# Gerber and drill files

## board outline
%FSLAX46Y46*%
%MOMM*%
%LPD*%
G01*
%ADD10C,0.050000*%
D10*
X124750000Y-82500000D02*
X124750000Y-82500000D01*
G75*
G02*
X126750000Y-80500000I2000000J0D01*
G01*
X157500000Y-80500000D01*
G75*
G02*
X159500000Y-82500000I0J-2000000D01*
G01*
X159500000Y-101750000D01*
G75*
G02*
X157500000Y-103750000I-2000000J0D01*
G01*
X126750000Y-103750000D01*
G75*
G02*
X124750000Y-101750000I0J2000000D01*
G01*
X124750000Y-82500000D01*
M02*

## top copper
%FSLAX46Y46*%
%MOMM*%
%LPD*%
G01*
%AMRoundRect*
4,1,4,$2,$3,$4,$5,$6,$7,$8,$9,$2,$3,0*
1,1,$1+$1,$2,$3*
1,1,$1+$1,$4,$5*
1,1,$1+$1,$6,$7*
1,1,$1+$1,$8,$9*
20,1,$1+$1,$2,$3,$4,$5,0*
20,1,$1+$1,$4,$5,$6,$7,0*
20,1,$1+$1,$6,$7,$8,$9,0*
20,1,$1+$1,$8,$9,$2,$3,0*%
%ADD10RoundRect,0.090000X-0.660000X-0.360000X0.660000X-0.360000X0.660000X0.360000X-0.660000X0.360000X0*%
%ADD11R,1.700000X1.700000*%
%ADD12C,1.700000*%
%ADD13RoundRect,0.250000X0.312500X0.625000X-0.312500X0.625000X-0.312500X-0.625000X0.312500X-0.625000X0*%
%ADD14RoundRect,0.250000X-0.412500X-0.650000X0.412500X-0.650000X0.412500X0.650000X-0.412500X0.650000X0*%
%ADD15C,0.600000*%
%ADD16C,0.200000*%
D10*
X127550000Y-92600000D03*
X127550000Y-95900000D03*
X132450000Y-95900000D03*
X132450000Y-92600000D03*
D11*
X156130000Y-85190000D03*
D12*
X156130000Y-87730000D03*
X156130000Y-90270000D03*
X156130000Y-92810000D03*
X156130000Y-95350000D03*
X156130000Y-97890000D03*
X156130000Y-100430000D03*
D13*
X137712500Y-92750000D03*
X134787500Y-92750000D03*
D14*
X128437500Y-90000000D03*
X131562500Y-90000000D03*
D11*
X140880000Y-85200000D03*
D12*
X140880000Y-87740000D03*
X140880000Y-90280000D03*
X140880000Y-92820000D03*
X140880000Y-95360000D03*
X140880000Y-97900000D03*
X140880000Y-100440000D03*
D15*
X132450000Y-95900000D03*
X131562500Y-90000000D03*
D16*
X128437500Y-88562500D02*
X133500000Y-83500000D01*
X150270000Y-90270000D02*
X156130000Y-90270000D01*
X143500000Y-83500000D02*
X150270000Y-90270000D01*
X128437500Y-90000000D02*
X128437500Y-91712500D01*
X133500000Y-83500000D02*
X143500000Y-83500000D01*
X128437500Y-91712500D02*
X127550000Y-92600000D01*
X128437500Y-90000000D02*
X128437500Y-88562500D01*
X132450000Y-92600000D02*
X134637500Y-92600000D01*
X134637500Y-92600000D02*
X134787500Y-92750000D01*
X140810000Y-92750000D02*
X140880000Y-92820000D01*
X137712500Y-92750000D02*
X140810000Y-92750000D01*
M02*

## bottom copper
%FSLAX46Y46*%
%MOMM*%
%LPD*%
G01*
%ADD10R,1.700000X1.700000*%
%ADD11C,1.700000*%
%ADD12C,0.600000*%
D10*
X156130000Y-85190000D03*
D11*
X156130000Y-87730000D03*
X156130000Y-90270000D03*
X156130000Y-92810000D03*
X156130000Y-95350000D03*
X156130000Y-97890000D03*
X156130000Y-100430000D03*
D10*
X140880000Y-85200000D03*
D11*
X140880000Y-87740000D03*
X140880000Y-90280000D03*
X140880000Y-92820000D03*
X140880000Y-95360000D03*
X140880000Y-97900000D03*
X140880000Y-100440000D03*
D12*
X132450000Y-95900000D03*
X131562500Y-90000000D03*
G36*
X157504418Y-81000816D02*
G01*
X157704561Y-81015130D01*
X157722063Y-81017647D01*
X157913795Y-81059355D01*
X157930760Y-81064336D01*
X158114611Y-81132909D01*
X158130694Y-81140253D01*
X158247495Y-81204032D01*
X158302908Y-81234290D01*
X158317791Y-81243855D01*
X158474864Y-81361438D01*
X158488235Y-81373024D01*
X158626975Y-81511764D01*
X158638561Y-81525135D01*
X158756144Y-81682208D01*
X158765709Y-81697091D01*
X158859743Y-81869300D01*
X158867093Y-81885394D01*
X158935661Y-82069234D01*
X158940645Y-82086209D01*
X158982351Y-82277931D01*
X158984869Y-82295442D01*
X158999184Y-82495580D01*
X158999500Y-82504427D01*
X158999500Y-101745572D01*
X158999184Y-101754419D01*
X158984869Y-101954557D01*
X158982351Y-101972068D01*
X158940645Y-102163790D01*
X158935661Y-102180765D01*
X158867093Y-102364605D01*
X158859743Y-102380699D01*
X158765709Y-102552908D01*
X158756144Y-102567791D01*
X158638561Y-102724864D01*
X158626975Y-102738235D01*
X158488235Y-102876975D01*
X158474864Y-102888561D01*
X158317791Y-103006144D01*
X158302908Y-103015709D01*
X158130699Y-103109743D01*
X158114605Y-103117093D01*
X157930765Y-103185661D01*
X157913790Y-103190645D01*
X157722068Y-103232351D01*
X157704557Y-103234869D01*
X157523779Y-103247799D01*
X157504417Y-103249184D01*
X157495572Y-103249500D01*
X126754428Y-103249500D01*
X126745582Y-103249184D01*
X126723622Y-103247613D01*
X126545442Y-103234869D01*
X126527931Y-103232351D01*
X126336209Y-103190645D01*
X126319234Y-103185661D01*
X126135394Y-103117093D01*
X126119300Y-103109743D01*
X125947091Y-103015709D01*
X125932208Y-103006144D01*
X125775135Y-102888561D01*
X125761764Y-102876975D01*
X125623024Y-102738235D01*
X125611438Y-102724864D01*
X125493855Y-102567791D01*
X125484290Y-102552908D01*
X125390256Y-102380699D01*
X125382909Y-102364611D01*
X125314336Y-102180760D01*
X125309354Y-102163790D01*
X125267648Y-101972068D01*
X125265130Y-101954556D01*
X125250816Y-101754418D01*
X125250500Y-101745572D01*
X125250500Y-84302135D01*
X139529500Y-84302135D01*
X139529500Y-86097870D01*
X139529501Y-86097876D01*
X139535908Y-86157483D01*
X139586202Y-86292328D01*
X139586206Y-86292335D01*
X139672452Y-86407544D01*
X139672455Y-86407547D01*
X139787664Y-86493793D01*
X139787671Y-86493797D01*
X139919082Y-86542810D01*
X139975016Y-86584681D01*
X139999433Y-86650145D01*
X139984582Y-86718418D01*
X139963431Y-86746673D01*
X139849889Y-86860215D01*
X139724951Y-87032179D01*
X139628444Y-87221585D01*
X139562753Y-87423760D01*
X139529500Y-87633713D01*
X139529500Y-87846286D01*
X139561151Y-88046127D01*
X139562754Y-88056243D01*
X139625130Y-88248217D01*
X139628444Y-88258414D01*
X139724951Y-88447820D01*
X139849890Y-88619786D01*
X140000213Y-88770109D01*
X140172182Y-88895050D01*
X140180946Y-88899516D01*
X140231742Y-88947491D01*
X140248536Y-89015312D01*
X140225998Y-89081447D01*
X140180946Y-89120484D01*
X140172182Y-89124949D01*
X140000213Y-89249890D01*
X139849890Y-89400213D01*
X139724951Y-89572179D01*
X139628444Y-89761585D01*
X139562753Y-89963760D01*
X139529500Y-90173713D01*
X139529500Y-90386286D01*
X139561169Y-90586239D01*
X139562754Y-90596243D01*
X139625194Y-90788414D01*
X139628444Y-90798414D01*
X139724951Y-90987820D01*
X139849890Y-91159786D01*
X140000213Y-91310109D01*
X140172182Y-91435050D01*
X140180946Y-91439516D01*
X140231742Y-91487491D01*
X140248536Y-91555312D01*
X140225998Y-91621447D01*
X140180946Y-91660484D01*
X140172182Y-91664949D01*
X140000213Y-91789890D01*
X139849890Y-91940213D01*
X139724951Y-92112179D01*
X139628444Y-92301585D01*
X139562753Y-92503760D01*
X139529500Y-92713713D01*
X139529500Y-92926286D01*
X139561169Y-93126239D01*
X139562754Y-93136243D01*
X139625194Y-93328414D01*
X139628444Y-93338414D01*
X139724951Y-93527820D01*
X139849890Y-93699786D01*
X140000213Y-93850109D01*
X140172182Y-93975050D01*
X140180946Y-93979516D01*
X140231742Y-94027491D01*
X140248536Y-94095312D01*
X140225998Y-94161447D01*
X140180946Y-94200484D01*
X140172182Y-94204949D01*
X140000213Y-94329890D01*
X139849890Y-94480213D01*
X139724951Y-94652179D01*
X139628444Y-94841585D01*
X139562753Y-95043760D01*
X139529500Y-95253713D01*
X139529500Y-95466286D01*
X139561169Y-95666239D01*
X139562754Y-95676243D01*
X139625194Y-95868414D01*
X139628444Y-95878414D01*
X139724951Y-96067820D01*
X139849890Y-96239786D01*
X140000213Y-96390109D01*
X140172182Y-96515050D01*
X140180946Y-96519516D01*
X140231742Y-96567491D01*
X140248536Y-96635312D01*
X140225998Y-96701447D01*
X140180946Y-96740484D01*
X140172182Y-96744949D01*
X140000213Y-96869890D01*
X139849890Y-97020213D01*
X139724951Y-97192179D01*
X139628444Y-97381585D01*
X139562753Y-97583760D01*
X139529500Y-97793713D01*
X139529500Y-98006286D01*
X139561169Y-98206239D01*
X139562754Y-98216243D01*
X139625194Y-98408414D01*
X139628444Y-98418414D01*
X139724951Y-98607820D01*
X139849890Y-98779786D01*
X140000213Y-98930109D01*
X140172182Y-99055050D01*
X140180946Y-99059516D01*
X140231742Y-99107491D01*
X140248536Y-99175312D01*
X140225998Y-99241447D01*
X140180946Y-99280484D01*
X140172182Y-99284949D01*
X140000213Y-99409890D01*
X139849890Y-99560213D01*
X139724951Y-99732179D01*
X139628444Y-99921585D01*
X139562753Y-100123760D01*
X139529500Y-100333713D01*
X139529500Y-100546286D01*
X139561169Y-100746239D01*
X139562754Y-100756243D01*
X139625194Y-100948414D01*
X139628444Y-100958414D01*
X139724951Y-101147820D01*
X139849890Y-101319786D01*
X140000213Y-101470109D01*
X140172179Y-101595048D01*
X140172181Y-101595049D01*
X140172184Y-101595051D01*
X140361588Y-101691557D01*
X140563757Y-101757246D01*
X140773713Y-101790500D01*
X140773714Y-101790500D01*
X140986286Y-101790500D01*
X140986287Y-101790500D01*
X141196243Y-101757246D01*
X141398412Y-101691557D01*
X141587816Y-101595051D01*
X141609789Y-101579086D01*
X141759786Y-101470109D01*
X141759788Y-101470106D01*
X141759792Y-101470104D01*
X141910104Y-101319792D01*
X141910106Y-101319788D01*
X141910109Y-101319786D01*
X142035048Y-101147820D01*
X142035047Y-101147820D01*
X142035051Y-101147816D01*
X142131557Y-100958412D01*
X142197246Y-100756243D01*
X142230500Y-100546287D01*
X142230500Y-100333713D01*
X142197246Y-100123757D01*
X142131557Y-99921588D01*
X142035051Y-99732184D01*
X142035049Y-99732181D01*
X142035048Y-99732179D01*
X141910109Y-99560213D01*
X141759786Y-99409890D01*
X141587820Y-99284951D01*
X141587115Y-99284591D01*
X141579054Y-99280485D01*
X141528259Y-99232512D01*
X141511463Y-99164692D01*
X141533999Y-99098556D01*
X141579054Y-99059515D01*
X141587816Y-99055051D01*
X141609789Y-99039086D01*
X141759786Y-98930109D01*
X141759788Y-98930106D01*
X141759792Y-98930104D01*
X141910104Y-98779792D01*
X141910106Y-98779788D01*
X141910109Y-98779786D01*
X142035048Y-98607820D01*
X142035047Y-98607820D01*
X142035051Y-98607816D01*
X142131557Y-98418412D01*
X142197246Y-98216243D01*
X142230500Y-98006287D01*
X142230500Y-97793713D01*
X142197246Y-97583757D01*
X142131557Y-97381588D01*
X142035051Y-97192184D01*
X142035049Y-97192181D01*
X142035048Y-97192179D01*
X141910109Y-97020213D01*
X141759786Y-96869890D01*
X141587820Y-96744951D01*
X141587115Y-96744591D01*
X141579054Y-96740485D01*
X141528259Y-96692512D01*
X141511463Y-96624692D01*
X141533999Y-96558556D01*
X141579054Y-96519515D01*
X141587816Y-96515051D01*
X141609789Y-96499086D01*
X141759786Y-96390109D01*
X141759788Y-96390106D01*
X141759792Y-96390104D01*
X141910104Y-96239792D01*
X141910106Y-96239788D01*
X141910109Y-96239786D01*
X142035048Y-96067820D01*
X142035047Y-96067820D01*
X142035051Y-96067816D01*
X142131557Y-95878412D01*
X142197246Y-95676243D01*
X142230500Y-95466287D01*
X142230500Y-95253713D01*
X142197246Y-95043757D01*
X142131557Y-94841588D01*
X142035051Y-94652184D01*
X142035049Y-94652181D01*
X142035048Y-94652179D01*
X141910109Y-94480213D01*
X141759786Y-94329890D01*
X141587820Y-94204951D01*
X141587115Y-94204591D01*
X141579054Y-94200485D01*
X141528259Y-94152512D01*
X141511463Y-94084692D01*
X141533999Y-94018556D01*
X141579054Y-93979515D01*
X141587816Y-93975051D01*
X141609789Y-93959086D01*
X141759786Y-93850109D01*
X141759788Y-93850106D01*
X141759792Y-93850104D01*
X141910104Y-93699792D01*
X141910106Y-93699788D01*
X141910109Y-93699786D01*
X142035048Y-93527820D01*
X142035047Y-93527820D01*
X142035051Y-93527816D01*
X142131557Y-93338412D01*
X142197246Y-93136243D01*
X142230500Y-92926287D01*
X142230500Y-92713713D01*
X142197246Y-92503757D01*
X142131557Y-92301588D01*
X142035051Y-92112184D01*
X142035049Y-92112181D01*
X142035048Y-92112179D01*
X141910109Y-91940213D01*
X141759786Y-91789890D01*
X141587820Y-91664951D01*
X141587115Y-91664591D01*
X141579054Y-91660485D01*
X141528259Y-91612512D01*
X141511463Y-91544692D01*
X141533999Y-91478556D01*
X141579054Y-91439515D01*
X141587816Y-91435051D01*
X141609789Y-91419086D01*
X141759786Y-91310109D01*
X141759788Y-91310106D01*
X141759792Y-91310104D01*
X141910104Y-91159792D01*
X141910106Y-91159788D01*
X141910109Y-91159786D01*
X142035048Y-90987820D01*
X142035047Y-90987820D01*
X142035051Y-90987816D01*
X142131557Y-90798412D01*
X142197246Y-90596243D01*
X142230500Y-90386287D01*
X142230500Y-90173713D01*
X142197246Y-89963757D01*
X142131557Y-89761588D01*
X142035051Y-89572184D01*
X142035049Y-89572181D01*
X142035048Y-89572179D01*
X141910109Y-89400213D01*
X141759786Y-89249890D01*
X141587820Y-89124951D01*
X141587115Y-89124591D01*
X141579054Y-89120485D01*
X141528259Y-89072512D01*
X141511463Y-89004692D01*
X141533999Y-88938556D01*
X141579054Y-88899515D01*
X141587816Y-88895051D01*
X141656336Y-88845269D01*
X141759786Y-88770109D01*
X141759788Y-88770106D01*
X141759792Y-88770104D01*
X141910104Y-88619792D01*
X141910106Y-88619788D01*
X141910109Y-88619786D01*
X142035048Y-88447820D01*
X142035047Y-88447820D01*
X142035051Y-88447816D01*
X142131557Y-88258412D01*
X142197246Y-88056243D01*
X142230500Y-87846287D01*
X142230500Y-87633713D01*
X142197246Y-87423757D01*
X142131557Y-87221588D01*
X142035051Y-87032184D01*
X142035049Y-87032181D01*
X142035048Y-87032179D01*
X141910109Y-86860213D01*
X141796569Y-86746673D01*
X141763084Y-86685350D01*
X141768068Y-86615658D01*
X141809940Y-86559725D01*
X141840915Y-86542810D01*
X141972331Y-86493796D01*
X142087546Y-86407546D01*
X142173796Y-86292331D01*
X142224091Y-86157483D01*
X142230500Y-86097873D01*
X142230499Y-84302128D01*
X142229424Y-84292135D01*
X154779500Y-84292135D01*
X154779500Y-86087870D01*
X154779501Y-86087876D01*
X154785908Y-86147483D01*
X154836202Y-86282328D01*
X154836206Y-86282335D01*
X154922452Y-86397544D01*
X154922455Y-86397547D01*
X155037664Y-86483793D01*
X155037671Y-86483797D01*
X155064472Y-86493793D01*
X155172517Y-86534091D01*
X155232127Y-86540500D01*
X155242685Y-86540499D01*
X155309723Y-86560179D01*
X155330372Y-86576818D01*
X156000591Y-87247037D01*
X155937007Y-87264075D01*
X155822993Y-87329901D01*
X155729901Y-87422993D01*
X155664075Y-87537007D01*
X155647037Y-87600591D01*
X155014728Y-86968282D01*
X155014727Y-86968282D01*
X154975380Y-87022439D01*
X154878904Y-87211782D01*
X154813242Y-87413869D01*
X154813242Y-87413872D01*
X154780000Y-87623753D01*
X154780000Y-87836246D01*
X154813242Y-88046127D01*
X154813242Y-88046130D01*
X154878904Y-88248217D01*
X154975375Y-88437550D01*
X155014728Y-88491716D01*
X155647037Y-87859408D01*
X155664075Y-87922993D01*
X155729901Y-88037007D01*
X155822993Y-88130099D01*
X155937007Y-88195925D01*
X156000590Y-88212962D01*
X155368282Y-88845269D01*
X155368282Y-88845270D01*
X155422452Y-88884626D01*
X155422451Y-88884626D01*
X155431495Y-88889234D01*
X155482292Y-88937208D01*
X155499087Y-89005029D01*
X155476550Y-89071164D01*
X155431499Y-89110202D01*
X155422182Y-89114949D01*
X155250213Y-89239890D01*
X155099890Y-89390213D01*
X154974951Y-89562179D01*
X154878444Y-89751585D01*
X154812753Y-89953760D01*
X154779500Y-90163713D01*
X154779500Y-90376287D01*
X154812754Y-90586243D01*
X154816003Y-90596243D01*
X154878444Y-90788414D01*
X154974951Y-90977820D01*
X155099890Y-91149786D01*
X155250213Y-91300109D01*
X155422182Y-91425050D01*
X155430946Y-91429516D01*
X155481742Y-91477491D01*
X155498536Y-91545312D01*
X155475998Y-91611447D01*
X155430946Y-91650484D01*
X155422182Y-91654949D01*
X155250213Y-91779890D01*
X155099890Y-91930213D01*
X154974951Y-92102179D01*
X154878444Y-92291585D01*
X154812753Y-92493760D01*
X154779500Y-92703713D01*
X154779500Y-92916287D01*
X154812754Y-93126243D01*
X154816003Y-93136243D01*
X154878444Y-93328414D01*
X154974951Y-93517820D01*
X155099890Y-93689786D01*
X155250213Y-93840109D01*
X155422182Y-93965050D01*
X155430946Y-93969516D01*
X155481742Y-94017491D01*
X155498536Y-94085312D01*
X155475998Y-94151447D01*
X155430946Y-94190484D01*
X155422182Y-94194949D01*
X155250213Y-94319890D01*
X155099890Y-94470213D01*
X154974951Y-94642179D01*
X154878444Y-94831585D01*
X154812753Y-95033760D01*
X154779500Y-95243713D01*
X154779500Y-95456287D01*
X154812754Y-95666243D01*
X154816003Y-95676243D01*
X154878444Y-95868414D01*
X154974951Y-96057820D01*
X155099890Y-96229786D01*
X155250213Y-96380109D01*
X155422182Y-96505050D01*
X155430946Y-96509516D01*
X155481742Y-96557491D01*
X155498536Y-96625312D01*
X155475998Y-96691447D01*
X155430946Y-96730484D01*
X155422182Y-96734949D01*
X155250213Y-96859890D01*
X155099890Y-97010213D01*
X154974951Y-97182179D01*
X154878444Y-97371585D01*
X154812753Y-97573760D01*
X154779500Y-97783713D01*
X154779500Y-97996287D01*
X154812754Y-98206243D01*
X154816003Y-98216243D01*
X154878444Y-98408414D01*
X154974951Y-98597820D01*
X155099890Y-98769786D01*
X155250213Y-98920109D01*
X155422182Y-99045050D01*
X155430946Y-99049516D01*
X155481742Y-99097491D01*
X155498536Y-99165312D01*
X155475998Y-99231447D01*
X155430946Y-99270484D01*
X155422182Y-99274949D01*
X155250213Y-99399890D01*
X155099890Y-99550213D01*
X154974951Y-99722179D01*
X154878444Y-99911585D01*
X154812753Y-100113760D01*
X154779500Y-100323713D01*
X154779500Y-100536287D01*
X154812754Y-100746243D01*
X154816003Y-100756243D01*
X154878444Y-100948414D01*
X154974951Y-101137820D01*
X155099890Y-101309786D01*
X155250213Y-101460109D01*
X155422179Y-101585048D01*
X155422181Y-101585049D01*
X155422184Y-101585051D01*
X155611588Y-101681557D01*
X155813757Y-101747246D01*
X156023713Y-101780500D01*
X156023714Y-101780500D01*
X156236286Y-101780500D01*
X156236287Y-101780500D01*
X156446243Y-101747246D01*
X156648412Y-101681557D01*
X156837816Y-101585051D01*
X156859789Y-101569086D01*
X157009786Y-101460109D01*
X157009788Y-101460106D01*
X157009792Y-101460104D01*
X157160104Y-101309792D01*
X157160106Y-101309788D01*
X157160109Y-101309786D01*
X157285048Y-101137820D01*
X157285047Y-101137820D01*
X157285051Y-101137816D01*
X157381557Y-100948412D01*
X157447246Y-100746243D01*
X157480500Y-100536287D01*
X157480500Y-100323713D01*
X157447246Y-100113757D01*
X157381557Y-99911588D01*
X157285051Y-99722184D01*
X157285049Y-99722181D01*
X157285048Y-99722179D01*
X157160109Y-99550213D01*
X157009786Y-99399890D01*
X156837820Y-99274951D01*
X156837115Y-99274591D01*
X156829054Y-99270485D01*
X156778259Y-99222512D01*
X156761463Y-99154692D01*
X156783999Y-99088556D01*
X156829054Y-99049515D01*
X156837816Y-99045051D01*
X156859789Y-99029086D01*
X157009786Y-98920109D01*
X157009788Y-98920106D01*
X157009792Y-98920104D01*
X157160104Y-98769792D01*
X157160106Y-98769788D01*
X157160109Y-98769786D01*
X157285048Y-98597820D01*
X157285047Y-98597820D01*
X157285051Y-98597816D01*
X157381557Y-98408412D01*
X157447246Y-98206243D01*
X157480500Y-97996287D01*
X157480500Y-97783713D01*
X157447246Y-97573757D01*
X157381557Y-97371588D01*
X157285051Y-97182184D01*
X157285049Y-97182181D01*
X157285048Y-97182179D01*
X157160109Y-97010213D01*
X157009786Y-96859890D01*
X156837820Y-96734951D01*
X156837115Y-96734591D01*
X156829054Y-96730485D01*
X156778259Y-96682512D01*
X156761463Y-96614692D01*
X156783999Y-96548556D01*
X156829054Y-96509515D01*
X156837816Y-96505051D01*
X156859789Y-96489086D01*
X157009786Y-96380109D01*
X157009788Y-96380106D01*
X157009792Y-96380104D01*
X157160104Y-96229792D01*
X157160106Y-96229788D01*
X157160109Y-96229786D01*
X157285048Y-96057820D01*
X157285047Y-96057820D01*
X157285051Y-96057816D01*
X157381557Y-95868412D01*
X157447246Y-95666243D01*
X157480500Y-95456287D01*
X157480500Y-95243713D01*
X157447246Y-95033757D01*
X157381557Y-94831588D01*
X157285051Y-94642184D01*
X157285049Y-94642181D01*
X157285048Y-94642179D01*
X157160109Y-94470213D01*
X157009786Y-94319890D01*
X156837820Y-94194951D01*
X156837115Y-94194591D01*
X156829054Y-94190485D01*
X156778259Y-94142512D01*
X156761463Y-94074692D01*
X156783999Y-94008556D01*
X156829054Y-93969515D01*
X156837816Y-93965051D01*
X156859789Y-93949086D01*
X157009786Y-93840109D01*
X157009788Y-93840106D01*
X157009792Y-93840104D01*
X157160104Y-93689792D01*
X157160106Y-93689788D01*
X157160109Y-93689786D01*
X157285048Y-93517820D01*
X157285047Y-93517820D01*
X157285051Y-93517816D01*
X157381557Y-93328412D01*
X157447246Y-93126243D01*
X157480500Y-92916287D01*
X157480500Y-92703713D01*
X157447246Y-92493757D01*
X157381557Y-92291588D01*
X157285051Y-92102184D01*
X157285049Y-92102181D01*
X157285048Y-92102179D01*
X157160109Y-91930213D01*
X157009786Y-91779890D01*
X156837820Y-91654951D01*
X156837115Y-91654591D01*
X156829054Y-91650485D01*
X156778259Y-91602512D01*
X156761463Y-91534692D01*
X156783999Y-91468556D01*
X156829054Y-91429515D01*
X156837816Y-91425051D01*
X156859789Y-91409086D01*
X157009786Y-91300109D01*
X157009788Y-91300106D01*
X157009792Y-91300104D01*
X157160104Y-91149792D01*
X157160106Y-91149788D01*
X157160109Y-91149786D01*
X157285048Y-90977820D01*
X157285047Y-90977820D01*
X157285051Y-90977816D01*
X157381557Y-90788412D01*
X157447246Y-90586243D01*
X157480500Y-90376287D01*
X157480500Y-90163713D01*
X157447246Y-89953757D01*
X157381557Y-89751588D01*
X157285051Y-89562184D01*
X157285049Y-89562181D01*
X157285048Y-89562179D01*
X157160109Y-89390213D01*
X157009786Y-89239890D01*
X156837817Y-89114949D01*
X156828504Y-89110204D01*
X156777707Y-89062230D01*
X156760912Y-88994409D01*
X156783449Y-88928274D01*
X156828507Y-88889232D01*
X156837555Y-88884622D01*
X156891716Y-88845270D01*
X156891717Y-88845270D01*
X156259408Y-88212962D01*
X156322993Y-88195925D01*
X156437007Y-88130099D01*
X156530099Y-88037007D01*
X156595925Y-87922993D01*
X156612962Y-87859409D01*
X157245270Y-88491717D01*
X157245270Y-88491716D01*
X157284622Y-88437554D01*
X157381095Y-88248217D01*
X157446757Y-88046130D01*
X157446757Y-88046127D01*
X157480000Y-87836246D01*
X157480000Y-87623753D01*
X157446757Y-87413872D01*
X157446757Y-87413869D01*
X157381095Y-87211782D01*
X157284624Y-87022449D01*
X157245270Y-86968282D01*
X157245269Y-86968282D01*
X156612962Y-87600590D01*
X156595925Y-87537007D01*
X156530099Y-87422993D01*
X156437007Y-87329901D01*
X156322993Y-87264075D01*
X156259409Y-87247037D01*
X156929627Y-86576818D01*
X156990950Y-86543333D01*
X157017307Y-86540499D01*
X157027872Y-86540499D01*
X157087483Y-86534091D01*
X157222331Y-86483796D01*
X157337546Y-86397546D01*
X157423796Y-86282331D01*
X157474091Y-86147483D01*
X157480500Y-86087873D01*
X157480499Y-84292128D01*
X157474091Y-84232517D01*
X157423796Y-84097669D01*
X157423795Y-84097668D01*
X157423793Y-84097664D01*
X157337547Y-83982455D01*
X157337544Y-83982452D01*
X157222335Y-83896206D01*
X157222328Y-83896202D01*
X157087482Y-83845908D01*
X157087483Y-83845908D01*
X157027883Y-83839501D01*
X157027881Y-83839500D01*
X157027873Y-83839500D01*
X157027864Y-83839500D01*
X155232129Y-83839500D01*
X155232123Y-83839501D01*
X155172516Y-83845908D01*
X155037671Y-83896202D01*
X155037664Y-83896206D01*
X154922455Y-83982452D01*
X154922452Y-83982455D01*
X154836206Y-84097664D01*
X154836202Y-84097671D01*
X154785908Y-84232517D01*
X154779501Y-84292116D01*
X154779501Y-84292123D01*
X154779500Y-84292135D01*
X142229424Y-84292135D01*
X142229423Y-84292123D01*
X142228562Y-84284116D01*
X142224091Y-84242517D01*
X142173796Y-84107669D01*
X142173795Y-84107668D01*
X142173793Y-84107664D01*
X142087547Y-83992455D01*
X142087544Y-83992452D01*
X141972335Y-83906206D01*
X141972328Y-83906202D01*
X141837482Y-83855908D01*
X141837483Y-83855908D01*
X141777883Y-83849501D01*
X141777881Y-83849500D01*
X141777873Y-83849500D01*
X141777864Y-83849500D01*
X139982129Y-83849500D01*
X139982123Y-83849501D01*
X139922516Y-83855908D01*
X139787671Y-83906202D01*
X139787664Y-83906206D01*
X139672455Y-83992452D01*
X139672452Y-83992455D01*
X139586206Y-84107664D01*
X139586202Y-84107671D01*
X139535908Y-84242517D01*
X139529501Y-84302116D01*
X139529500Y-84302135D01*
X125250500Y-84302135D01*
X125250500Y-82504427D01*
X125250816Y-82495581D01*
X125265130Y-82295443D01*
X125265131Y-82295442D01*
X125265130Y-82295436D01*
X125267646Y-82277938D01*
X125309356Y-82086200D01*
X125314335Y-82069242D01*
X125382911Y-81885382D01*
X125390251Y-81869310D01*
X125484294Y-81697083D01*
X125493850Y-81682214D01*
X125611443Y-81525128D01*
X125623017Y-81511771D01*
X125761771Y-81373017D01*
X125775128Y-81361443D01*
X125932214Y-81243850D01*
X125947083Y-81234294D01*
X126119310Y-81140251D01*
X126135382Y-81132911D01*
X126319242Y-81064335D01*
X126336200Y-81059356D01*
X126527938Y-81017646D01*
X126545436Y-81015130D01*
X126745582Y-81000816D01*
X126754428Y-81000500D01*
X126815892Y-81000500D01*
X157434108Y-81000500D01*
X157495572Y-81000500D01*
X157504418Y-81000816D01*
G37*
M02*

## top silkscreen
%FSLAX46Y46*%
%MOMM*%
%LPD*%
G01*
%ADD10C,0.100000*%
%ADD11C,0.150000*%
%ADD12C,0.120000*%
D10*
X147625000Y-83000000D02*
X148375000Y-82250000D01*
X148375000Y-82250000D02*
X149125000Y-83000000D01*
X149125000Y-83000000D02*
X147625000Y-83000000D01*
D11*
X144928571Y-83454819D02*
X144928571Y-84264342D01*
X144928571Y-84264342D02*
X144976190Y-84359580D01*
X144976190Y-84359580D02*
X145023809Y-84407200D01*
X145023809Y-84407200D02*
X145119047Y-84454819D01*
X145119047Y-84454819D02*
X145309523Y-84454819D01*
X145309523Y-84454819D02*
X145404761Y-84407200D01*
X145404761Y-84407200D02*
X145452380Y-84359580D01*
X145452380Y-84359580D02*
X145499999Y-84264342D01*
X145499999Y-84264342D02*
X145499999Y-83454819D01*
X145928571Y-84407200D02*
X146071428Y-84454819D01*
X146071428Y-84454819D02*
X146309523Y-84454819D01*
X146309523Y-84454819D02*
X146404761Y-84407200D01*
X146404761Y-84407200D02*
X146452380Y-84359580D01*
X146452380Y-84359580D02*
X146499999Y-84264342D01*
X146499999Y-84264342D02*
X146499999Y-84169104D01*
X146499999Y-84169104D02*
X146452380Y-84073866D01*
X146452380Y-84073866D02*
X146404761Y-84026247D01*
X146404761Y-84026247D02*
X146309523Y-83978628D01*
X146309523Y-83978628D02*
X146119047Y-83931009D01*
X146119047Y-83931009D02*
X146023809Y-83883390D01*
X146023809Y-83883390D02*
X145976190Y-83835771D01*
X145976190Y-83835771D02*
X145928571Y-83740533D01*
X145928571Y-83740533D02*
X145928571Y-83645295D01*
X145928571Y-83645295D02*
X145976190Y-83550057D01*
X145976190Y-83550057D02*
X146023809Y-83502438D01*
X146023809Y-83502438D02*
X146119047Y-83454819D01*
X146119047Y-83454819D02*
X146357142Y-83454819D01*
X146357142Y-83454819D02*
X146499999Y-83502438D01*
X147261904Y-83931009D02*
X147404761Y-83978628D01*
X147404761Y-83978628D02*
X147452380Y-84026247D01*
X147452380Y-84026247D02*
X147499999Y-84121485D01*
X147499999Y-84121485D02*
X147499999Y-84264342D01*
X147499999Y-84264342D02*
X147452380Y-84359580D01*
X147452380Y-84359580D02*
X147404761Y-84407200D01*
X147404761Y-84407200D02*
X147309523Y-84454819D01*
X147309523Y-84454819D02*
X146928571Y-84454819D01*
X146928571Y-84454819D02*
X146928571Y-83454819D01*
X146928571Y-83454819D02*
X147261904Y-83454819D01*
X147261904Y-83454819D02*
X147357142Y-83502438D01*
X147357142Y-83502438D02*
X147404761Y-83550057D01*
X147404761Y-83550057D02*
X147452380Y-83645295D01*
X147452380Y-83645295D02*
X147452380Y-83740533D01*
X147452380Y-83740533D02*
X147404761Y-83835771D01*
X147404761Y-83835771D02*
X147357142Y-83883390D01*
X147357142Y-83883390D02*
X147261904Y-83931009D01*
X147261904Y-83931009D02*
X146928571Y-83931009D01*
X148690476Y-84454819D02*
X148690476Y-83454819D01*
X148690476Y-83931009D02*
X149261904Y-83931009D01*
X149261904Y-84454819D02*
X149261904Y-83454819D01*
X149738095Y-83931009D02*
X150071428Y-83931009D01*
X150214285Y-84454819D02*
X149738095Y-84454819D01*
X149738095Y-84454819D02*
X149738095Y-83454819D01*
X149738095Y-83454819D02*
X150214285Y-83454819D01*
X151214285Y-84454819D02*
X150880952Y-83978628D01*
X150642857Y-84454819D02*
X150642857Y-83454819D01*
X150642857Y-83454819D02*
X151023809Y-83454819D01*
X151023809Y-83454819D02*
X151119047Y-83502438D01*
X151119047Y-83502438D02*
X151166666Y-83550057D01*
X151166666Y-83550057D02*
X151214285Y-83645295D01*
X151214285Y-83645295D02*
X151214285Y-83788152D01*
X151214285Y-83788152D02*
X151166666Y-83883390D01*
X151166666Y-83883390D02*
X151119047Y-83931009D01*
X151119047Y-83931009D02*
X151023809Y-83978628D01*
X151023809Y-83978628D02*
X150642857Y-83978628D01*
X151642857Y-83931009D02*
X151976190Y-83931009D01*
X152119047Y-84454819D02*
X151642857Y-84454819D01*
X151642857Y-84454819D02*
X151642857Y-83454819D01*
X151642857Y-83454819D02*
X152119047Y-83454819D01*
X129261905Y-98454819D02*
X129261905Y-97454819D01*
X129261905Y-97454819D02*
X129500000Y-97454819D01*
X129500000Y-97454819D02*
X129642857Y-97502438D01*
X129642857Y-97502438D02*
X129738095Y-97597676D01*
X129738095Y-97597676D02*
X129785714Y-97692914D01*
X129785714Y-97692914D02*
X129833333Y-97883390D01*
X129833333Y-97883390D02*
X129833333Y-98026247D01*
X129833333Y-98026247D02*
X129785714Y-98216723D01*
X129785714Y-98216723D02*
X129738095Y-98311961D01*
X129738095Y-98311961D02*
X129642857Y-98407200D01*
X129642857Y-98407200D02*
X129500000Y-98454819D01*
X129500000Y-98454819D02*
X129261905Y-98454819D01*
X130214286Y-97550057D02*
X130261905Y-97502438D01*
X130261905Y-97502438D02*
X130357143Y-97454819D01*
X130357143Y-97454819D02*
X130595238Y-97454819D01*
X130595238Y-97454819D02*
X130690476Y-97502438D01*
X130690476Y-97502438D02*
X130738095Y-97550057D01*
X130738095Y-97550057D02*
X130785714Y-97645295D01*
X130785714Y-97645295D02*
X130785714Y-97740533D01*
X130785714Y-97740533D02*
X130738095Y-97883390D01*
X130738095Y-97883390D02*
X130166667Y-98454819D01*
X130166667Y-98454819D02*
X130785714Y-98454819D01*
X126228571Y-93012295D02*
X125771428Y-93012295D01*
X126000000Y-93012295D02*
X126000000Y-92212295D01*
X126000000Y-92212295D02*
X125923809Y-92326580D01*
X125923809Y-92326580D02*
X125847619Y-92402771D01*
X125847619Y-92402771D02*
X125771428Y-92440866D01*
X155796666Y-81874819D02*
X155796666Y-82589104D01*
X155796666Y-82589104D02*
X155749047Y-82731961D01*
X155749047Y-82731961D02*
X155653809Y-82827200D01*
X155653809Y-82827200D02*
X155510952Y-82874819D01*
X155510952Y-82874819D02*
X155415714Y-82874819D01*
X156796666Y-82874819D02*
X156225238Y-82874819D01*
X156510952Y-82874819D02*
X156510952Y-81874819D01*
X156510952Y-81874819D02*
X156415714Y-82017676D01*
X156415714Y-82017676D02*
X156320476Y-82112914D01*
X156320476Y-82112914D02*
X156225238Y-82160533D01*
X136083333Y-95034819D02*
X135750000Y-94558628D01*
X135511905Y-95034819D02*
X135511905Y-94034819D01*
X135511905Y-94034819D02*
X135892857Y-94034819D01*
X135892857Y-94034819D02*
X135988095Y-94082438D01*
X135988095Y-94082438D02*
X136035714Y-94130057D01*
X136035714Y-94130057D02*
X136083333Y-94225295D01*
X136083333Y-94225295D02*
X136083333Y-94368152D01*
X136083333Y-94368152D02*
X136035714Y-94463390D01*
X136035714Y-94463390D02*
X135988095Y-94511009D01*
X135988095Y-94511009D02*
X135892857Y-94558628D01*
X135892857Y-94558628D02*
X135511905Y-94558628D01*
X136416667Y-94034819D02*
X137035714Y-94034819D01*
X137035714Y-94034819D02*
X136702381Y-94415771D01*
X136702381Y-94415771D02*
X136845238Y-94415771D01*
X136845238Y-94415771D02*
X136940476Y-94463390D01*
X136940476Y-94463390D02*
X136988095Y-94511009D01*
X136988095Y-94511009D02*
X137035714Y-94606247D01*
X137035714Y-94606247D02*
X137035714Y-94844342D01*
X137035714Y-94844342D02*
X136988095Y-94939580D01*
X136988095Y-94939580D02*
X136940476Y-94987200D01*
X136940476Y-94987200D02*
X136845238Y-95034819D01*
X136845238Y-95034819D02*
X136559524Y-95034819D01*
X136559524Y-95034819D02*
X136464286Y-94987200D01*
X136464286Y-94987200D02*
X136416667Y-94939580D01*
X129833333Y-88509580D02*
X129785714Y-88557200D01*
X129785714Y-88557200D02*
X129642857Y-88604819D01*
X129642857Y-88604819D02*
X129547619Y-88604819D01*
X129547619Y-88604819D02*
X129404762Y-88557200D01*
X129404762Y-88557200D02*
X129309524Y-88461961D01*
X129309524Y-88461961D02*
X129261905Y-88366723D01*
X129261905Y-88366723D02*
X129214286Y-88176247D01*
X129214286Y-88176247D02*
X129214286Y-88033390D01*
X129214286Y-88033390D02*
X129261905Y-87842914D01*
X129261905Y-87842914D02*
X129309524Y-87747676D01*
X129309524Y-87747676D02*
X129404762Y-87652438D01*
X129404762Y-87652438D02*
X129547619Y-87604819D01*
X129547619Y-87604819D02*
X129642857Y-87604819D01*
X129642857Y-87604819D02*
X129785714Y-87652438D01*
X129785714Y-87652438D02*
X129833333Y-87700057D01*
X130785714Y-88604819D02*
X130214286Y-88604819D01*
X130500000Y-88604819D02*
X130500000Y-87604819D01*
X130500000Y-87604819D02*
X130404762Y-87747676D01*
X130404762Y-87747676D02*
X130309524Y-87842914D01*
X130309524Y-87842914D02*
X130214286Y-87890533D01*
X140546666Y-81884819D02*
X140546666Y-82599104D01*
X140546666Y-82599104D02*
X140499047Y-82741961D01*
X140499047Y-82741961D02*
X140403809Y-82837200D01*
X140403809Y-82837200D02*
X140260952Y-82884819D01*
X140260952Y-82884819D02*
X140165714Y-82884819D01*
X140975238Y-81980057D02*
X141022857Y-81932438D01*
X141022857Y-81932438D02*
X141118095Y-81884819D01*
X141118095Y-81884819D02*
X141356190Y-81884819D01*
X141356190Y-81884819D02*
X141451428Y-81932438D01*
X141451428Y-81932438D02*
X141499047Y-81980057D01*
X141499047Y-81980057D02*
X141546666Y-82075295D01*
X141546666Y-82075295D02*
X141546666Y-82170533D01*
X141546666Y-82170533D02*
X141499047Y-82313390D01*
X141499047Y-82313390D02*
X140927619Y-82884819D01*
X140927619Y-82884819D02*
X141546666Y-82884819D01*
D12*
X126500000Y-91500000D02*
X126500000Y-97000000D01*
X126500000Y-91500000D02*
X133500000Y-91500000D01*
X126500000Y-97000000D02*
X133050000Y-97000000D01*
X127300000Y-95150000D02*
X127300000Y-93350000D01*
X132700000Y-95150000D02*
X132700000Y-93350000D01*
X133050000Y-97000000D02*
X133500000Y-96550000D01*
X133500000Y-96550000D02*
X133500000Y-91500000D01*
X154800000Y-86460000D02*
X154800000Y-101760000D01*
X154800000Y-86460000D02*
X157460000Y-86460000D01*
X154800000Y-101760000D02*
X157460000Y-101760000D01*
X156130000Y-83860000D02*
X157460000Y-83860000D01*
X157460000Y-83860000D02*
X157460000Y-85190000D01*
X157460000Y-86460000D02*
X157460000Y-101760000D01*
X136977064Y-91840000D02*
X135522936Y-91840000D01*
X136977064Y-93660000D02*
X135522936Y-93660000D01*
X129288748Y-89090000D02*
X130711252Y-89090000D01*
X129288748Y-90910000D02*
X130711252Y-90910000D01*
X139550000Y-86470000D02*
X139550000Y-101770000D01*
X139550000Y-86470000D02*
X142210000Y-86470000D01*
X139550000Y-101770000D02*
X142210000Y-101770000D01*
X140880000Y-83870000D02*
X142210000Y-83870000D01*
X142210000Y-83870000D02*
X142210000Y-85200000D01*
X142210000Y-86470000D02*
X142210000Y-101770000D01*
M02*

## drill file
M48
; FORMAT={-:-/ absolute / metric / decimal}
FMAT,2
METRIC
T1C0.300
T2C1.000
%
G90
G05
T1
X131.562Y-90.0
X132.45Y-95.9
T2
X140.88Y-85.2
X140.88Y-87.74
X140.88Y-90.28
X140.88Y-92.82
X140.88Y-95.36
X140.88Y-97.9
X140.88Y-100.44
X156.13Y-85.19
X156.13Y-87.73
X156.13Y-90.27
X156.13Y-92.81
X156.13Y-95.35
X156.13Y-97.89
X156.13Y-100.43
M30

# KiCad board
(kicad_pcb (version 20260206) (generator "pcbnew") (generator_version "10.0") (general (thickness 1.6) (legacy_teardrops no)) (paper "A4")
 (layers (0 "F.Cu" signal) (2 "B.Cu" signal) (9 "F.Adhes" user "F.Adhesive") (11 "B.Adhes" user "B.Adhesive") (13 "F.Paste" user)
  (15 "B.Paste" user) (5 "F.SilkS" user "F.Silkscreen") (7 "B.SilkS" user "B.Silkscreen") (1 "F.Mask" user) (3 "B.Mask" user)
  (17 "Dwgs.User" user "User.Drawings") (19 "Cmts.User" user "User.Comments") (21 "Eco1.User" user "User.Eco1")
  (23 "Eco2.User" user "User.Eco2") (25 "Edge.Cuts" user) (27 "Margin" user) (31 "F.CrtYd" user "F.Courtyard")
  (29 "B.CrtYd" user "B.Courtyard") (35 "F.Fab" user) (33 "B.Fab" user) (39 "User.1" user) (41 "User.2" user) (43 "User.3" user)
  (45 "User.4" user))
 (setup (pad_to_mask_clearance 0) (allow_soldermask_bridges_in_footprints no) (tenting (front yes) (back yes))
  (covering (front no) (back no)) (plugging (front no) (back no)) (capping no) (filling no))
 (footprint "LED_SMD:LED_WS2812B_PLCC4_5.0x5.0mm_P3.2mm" (layer "F.Cu") (at 130 94.25)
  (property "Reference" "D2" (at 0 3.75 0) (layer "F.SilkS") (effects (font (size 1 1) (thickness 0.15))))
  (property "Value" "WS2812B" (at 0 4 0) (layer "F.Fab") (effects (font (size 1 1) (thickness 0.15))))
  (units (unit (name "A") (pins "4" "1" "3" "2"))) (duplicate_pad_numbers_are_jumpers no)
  (fp_line (start -3.5 -2.75) (end -3.5 2.75) (stroke (width 0.12) (type default)) (layer "F.SilkS"))
  (fp_line (start -3.5 -2.75) (end 3.5 -2.75) (stroke (width 0.12) (type solid)) (layer "F.SilkS"))
  (fp_line (start -3.5 2.75) (end 3.05 2.75) (stroke (width 0.12) (type solid)) (layer "F.SilkS"))
  (fp_line (start -2.7 0.9) (end -2.7 -0.9) (stroke (width 0.12) (type default)) (layer "F.SilkS"))
  (fp_line (start 2.7 0.9) (end 2.7 -0.9) (stroke (width 0.12) (type default)) (layer "F.SilkS"))
  (fp_line (start 3.05 2.75) (end 3.5 2.3) (stroke (width 0.12) (type default)) (layer "F.SilkS"))
  (fp_line (start 3.5 2.3) (end 3.5 -2.75) (stroke (width 0.12) (type default)) (layer "F.SilkS"))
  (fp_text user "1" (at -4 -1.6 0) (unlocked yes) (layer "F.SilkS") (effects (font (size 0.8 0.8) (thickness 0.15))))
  (pad "1" smd roundrect (at -2.45 -1.65) (size 1.5 0.9) (layers "F.Cu" "F.Mask" "F.Paste") (roundrect_rratio 0.1) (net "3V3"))
  (pad "2" smd roundrect (at -2.45 1.65) (size 1.5 0.9) (layers "F.Cu" "F.Mask" "F.Paste") (roundrect_rratio 0.1)
   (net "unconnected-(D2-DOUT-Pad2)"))
  (pad "3" smd roundrect (at 2.45 1.65) (size 1.5 0.9) (layers "F.Cu" "F.Mask" "F.Paste") (roundrect_rratio 0.1) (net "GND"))
  (pad "4" smd roundrect (at 2.45 -1.65) (size 1.5 0.9) (layers "F.Cu" "F.Mask" "F.Paste") (roundrect_rratio 0.1) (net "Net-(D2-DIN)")))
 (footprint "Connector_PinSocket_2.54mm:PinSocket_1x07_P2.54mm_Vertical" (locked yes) (layer "F.Cu") (at 156.13 85.19)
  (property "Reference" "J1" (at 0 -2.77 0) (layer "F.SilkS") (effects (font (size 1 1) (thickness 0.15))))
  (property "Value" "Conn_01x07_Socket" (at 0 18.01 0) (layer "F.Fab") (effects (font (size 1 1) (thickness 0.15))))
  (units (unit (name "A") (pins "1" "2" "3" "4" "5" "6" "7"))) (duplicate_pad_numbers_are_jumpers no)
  (fp_line (start -1.33 1.27) (end -1.33 16.57) (stroke (width 0.12) (type solid)) (layer "F.SilkS"))
  (fp_line (start -1.33 1.27) (end 1.33 1.27) (stroke (width 0.12) (type solid)) (layer "F.SilkS"))
  (fp_line (start -1.33 16.57) (end 1.33 16.57) (stroke (width 0.12) (type solid)) (layer "F.SilkS"))
  (fp_line (start 0 -1.33) (end 1.33 -1.33) (stroke (width 0.12) (type solid)) (layer "F.SilkS"))
  (fp_line (start 1.33 -1.33) (end 1.33 0) (stroke (width 0.12) (type solid)) (layer "F.SilkS"))
  (fp_line (start 1.33 1.27) (end 1.33 16.57) (stroke (width 0.12) (type solid)) (layer "F.SilkS"))
  (pad "1" thru_hole rect (at 0 0) (size 1.7 1.7) (drill 1) (layers "*.Cu" "*.Mask") (remove_unused_layers no)
   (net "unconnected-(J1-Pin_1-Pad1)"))
  (pad "2" thru_hole circle (at 0 2.54) (size 1.7 1.7) (drill 1) (layers "*.Cu" "*.Mask") (remove_unused_layers no) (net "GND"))
  (pad "3" thru_hole circle (at 0 5.08) (size 1.7 1.7) (drill 1) (layers "*.Cu" "*.Mask") (remove_unused_layers no) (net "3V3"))
  (pad "4" thru_hole circle (at 0 7.62) (size 1.7 1.7) (drill 1) (layers "*.Cu" "*.Mask") (remove_unused_layers no)
   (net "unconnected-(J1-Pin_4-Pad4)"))
  (pad "5" thru_hole circle (at 0 10.16) (size 1.7 1.7) (drill 1) (layers "*.Cu" "*.Mask") (remove_unused_layers no)
   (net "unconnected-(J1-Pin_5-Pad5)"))
  (pad "6" thru_hole circle (at 0 12.7) (size 1.7 1.7) (drill 1) (layers "*.Cu" "*.Mask") (remove_unused_layers no)
   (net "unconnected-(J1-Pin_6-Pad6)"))
  (pad "7" thru_hole circle (at 0 15.24) (size 1.7 1.7) (drill 1) (layers "*.Cu" "*.Mask") (remove_unused_layers no)
   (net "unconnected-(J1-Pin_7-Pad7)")))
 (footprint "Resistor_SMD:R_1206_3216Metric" (layer "F.Cu") (at 136.25 92.75 180)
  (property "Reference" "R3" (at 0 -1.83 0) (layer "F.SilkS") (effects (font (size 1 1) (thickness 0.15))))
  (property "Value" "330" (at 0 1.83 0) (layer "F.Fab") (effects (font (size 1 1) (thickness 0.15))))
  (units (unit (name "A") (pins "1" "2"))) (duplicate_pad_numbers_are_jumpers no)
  (fp_line (start -0.727064 0.91) (end 0.727064 0.91) (stroke (width 0.12) (type solid)) (layer "F.SilkS"))
  (fp_line (start -0.727064 -0.91) (end 0.727064 -0.91) (stroke (width 0.12) (type solid)) (layer "F.SilkS"))
  (pad "1" smd roundrect (at -1.4625 0 180) (size 1.125 1.75) (layers "F.Cu" "F.Mask" "F.Paste") (roundrect_rratio 0.222222) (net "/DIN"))
  (pad "2" smd roundrect (at 1.4625 0 180) (size 1.125 1.75) (layers "F.Cu" "F.Mask" "F.Paste") (roundrect_rratio 0.222222)
   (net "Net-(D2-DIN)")))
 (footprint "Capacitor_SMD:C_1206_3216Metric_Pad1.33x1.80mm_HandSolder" (layer "F.Cu") (at 130 90)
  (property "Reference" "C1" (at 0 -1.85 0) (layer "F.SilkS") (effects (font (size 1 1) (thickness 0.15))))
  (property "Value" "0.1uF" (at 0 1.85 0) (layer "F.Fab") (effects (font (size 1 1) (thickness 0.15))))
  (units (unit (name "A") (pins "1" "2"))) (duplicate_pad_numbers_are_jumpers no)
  (fp_line (start -0.711252 -0.91) (end 0.711252 -0.91) (stroke (width 0.12) (type solid)) (layer "F.SilkS"))
  (fp_line (start -0.711252 0.91) (end 0.711252 0.91) (stroke (width 0.12) (type solid)) (layer "F.SilkS"))
  (pad "1" smd roundrect (at -1.5625 0) (size 1.325 1.8) (layers "F.Cu" "F.Mask" "F.Paste") (roundrect_rratio 0.188679) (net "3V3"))
  (pad "2" smd roundrect (at 1.5625 0) (size 1.325 1.8) (layers "F.Cu" "F.Mask" "F.Paste") (roundrect_rratio 0.188679) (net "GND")))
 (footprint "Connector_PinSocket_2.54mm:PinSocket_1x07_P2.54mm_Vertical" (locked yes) (layer "F.Cu") (at 140.88 85.2)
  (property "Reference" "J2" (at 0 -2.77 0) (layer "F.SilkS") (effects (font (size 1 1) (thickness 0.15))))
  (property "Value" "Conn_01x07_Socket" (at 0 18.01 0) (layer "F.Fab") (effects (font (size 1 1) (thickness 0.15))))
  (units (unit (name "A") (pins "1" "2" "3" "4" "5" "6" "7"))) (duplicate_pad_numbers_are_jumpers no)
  (fp_line (start -1.33 1.27) (end -1.33 16.57) (stroke (width 0.12) (type solid)) (layer "F.SilkS"))
  (fp_line (start -1.33 1.27) (end 1.33 1.27) (stroke (width 0.12) (type solid)) (layer "F.SilkS"))
  (fp_line (start -1.33 16.57) (end 1.33 16.57) (stroke (width 0.12) (type solid)) (layer "F.SilkS"))
  (fp_line (start 0 -1.33) (end 1.33 -1.33) (stroke (width 0.12) (type solid)) (layer "F.SilkS"))
  (fp_line (start 1.33 -1.33) (end 1.33 0) (stroke (width 0.12) (type solid)) (layer "F.SilkS"))
  (fp_line (start 1.33 1.27) (end 1.33 16.57) (stroke (width 0.12) (type solid)) (layer "F.SilkS"))
  (pad "1" thru_hole rect (at 0 0) (size 1.7 1.7) (drill 1) (layers "*.Cu" "*.Mask") (remove_unused_layers no)
   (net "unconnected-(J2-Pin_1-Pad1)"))
  (pad "2" thru_hole circle (at 0 2.54) (size 1.7 1.7) (drill 1) (layers "*.Cu" "*.Mask") (remove_unused_layers no)
   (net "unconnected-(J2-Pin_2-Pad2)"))
  (pad "3" thru_hole circle (at 0 5.08) (size 1.7 1.7) (drill 1) (layers "*.Cu" "*.Mask") (remove_unused_layers no)
   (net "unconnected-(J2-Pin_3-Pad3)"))
  (pad "4" thru_hole circle (at 0 7.62) (size 1.7 1.7) (drill 1) (layers "*.Cu" "*.Mask") (remove_unused_layers no) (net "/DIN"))
  (pad "5" thru_hole circle (at 0 10.16) (size 1.7 1.7) (drill 1) (layers "*.Cu" "*.Mask") (remove_unused_layers no)
   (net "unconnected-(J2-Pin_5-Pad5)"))
  (pad "6" thru_hole circle (at 0 12.7) (size 1.7 1.7) (drill 1) (layers "*.Cu" "*.Mask") (remove_unused_layers no)
   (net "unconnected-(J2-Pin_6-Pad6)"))
  (pad "7" thru_hole circle (at 0 15.24) (size 1.7 1.7) (drill 1) (layers "*.Cu" "*.Mask") (remove_unused_layers no)
   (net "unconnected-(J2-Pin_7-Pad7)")))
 (gr_line (start 147.625 83) (end 148.375 82.25) (stroke (width 0.1) (type default)) (layer "F.SilkS"))
 (gr_line (start 148.375 82.25) (end 149.125 83) (stroke (width 0.1) (type default)) (layer "F.SilkS"))
 (gr_line (start 149.125 83) (end 147.625 83) (stroke (width 0.1) (type default)) (layer "F.SilkS"))
 (gr_rect (start 124.75 80.5) (end 159.5 103.75) (radius 2) (stroke (width 0.05) (type solid)) (fill no) (layer "Edge.Cuts"))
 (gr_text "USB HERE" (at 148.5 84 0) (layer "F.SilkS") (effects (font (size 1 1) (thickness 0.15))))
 (segment (start 128.4375 88.5625) (end 133.5 83.5) (width 0.2) (layer "F.Cu") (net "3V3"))
 (segment (start 150.27 90.27) (end 156.13 90.27) (width 0.2) (layer "F.Cu") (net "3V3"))
 (segment (start 143.5 83.5) (end 150.27 90.27) (width 0.2) (layer "F.Cu") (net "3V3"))
 (segment (start 128.4375 90) (end 128.4375 91.7125) (width 0.2) (layer "F.Cu") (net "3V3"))
 (segment (start 133.5 83.5) (end 143.5 83.5) (width 0.2) (layer "F.Cu") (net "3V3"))
 (segment (start 128.4375 91.7125) (end 127.55 92.6) (width 0.2) (layer "F.Cu") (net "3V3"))
 (segment (start 128.4375 90) (end 128.4375 88.5625) (width 0.2) (layer "F.Cu") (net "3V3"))
 (via (at 132.45 95.9) (size 0.6) (drill 0.3) (layers "F.Cu" "B.Cu") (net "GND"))
 (via (at 131.5625 90) (size 0.6) (drill 0.3) (layers "F.Cu" "B.Cu") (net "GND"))
 (segment (start 132.45 92.6) (end 134.6375 92.6) (width 0.2) (layer "F.Cu") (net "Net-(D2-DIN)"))
 (segment (start 134.6375 92.6) (end 134.7875 92.75) (width 0.2) (layer "F.Cu") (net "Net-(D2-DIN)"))
 (segment (start 140.81 92.75) (end 140.88 92.82) (width 0.2) (locked yes) (layer "F.Cu") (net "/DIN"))
 (segment (start 137.7125 92.75) (end 140.81 92.75) (width 0.2) (layer "F.Cu") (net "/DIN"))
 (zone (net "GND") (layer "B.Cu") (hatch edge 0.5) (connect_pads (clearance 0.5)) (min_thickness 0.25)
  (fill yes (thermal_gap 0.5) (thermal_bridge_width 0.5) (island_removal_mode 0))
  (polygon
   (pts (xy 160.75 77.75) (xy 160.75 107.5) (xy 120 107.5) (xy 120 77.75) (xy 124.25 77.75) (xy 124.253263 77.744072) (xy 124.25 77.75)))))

